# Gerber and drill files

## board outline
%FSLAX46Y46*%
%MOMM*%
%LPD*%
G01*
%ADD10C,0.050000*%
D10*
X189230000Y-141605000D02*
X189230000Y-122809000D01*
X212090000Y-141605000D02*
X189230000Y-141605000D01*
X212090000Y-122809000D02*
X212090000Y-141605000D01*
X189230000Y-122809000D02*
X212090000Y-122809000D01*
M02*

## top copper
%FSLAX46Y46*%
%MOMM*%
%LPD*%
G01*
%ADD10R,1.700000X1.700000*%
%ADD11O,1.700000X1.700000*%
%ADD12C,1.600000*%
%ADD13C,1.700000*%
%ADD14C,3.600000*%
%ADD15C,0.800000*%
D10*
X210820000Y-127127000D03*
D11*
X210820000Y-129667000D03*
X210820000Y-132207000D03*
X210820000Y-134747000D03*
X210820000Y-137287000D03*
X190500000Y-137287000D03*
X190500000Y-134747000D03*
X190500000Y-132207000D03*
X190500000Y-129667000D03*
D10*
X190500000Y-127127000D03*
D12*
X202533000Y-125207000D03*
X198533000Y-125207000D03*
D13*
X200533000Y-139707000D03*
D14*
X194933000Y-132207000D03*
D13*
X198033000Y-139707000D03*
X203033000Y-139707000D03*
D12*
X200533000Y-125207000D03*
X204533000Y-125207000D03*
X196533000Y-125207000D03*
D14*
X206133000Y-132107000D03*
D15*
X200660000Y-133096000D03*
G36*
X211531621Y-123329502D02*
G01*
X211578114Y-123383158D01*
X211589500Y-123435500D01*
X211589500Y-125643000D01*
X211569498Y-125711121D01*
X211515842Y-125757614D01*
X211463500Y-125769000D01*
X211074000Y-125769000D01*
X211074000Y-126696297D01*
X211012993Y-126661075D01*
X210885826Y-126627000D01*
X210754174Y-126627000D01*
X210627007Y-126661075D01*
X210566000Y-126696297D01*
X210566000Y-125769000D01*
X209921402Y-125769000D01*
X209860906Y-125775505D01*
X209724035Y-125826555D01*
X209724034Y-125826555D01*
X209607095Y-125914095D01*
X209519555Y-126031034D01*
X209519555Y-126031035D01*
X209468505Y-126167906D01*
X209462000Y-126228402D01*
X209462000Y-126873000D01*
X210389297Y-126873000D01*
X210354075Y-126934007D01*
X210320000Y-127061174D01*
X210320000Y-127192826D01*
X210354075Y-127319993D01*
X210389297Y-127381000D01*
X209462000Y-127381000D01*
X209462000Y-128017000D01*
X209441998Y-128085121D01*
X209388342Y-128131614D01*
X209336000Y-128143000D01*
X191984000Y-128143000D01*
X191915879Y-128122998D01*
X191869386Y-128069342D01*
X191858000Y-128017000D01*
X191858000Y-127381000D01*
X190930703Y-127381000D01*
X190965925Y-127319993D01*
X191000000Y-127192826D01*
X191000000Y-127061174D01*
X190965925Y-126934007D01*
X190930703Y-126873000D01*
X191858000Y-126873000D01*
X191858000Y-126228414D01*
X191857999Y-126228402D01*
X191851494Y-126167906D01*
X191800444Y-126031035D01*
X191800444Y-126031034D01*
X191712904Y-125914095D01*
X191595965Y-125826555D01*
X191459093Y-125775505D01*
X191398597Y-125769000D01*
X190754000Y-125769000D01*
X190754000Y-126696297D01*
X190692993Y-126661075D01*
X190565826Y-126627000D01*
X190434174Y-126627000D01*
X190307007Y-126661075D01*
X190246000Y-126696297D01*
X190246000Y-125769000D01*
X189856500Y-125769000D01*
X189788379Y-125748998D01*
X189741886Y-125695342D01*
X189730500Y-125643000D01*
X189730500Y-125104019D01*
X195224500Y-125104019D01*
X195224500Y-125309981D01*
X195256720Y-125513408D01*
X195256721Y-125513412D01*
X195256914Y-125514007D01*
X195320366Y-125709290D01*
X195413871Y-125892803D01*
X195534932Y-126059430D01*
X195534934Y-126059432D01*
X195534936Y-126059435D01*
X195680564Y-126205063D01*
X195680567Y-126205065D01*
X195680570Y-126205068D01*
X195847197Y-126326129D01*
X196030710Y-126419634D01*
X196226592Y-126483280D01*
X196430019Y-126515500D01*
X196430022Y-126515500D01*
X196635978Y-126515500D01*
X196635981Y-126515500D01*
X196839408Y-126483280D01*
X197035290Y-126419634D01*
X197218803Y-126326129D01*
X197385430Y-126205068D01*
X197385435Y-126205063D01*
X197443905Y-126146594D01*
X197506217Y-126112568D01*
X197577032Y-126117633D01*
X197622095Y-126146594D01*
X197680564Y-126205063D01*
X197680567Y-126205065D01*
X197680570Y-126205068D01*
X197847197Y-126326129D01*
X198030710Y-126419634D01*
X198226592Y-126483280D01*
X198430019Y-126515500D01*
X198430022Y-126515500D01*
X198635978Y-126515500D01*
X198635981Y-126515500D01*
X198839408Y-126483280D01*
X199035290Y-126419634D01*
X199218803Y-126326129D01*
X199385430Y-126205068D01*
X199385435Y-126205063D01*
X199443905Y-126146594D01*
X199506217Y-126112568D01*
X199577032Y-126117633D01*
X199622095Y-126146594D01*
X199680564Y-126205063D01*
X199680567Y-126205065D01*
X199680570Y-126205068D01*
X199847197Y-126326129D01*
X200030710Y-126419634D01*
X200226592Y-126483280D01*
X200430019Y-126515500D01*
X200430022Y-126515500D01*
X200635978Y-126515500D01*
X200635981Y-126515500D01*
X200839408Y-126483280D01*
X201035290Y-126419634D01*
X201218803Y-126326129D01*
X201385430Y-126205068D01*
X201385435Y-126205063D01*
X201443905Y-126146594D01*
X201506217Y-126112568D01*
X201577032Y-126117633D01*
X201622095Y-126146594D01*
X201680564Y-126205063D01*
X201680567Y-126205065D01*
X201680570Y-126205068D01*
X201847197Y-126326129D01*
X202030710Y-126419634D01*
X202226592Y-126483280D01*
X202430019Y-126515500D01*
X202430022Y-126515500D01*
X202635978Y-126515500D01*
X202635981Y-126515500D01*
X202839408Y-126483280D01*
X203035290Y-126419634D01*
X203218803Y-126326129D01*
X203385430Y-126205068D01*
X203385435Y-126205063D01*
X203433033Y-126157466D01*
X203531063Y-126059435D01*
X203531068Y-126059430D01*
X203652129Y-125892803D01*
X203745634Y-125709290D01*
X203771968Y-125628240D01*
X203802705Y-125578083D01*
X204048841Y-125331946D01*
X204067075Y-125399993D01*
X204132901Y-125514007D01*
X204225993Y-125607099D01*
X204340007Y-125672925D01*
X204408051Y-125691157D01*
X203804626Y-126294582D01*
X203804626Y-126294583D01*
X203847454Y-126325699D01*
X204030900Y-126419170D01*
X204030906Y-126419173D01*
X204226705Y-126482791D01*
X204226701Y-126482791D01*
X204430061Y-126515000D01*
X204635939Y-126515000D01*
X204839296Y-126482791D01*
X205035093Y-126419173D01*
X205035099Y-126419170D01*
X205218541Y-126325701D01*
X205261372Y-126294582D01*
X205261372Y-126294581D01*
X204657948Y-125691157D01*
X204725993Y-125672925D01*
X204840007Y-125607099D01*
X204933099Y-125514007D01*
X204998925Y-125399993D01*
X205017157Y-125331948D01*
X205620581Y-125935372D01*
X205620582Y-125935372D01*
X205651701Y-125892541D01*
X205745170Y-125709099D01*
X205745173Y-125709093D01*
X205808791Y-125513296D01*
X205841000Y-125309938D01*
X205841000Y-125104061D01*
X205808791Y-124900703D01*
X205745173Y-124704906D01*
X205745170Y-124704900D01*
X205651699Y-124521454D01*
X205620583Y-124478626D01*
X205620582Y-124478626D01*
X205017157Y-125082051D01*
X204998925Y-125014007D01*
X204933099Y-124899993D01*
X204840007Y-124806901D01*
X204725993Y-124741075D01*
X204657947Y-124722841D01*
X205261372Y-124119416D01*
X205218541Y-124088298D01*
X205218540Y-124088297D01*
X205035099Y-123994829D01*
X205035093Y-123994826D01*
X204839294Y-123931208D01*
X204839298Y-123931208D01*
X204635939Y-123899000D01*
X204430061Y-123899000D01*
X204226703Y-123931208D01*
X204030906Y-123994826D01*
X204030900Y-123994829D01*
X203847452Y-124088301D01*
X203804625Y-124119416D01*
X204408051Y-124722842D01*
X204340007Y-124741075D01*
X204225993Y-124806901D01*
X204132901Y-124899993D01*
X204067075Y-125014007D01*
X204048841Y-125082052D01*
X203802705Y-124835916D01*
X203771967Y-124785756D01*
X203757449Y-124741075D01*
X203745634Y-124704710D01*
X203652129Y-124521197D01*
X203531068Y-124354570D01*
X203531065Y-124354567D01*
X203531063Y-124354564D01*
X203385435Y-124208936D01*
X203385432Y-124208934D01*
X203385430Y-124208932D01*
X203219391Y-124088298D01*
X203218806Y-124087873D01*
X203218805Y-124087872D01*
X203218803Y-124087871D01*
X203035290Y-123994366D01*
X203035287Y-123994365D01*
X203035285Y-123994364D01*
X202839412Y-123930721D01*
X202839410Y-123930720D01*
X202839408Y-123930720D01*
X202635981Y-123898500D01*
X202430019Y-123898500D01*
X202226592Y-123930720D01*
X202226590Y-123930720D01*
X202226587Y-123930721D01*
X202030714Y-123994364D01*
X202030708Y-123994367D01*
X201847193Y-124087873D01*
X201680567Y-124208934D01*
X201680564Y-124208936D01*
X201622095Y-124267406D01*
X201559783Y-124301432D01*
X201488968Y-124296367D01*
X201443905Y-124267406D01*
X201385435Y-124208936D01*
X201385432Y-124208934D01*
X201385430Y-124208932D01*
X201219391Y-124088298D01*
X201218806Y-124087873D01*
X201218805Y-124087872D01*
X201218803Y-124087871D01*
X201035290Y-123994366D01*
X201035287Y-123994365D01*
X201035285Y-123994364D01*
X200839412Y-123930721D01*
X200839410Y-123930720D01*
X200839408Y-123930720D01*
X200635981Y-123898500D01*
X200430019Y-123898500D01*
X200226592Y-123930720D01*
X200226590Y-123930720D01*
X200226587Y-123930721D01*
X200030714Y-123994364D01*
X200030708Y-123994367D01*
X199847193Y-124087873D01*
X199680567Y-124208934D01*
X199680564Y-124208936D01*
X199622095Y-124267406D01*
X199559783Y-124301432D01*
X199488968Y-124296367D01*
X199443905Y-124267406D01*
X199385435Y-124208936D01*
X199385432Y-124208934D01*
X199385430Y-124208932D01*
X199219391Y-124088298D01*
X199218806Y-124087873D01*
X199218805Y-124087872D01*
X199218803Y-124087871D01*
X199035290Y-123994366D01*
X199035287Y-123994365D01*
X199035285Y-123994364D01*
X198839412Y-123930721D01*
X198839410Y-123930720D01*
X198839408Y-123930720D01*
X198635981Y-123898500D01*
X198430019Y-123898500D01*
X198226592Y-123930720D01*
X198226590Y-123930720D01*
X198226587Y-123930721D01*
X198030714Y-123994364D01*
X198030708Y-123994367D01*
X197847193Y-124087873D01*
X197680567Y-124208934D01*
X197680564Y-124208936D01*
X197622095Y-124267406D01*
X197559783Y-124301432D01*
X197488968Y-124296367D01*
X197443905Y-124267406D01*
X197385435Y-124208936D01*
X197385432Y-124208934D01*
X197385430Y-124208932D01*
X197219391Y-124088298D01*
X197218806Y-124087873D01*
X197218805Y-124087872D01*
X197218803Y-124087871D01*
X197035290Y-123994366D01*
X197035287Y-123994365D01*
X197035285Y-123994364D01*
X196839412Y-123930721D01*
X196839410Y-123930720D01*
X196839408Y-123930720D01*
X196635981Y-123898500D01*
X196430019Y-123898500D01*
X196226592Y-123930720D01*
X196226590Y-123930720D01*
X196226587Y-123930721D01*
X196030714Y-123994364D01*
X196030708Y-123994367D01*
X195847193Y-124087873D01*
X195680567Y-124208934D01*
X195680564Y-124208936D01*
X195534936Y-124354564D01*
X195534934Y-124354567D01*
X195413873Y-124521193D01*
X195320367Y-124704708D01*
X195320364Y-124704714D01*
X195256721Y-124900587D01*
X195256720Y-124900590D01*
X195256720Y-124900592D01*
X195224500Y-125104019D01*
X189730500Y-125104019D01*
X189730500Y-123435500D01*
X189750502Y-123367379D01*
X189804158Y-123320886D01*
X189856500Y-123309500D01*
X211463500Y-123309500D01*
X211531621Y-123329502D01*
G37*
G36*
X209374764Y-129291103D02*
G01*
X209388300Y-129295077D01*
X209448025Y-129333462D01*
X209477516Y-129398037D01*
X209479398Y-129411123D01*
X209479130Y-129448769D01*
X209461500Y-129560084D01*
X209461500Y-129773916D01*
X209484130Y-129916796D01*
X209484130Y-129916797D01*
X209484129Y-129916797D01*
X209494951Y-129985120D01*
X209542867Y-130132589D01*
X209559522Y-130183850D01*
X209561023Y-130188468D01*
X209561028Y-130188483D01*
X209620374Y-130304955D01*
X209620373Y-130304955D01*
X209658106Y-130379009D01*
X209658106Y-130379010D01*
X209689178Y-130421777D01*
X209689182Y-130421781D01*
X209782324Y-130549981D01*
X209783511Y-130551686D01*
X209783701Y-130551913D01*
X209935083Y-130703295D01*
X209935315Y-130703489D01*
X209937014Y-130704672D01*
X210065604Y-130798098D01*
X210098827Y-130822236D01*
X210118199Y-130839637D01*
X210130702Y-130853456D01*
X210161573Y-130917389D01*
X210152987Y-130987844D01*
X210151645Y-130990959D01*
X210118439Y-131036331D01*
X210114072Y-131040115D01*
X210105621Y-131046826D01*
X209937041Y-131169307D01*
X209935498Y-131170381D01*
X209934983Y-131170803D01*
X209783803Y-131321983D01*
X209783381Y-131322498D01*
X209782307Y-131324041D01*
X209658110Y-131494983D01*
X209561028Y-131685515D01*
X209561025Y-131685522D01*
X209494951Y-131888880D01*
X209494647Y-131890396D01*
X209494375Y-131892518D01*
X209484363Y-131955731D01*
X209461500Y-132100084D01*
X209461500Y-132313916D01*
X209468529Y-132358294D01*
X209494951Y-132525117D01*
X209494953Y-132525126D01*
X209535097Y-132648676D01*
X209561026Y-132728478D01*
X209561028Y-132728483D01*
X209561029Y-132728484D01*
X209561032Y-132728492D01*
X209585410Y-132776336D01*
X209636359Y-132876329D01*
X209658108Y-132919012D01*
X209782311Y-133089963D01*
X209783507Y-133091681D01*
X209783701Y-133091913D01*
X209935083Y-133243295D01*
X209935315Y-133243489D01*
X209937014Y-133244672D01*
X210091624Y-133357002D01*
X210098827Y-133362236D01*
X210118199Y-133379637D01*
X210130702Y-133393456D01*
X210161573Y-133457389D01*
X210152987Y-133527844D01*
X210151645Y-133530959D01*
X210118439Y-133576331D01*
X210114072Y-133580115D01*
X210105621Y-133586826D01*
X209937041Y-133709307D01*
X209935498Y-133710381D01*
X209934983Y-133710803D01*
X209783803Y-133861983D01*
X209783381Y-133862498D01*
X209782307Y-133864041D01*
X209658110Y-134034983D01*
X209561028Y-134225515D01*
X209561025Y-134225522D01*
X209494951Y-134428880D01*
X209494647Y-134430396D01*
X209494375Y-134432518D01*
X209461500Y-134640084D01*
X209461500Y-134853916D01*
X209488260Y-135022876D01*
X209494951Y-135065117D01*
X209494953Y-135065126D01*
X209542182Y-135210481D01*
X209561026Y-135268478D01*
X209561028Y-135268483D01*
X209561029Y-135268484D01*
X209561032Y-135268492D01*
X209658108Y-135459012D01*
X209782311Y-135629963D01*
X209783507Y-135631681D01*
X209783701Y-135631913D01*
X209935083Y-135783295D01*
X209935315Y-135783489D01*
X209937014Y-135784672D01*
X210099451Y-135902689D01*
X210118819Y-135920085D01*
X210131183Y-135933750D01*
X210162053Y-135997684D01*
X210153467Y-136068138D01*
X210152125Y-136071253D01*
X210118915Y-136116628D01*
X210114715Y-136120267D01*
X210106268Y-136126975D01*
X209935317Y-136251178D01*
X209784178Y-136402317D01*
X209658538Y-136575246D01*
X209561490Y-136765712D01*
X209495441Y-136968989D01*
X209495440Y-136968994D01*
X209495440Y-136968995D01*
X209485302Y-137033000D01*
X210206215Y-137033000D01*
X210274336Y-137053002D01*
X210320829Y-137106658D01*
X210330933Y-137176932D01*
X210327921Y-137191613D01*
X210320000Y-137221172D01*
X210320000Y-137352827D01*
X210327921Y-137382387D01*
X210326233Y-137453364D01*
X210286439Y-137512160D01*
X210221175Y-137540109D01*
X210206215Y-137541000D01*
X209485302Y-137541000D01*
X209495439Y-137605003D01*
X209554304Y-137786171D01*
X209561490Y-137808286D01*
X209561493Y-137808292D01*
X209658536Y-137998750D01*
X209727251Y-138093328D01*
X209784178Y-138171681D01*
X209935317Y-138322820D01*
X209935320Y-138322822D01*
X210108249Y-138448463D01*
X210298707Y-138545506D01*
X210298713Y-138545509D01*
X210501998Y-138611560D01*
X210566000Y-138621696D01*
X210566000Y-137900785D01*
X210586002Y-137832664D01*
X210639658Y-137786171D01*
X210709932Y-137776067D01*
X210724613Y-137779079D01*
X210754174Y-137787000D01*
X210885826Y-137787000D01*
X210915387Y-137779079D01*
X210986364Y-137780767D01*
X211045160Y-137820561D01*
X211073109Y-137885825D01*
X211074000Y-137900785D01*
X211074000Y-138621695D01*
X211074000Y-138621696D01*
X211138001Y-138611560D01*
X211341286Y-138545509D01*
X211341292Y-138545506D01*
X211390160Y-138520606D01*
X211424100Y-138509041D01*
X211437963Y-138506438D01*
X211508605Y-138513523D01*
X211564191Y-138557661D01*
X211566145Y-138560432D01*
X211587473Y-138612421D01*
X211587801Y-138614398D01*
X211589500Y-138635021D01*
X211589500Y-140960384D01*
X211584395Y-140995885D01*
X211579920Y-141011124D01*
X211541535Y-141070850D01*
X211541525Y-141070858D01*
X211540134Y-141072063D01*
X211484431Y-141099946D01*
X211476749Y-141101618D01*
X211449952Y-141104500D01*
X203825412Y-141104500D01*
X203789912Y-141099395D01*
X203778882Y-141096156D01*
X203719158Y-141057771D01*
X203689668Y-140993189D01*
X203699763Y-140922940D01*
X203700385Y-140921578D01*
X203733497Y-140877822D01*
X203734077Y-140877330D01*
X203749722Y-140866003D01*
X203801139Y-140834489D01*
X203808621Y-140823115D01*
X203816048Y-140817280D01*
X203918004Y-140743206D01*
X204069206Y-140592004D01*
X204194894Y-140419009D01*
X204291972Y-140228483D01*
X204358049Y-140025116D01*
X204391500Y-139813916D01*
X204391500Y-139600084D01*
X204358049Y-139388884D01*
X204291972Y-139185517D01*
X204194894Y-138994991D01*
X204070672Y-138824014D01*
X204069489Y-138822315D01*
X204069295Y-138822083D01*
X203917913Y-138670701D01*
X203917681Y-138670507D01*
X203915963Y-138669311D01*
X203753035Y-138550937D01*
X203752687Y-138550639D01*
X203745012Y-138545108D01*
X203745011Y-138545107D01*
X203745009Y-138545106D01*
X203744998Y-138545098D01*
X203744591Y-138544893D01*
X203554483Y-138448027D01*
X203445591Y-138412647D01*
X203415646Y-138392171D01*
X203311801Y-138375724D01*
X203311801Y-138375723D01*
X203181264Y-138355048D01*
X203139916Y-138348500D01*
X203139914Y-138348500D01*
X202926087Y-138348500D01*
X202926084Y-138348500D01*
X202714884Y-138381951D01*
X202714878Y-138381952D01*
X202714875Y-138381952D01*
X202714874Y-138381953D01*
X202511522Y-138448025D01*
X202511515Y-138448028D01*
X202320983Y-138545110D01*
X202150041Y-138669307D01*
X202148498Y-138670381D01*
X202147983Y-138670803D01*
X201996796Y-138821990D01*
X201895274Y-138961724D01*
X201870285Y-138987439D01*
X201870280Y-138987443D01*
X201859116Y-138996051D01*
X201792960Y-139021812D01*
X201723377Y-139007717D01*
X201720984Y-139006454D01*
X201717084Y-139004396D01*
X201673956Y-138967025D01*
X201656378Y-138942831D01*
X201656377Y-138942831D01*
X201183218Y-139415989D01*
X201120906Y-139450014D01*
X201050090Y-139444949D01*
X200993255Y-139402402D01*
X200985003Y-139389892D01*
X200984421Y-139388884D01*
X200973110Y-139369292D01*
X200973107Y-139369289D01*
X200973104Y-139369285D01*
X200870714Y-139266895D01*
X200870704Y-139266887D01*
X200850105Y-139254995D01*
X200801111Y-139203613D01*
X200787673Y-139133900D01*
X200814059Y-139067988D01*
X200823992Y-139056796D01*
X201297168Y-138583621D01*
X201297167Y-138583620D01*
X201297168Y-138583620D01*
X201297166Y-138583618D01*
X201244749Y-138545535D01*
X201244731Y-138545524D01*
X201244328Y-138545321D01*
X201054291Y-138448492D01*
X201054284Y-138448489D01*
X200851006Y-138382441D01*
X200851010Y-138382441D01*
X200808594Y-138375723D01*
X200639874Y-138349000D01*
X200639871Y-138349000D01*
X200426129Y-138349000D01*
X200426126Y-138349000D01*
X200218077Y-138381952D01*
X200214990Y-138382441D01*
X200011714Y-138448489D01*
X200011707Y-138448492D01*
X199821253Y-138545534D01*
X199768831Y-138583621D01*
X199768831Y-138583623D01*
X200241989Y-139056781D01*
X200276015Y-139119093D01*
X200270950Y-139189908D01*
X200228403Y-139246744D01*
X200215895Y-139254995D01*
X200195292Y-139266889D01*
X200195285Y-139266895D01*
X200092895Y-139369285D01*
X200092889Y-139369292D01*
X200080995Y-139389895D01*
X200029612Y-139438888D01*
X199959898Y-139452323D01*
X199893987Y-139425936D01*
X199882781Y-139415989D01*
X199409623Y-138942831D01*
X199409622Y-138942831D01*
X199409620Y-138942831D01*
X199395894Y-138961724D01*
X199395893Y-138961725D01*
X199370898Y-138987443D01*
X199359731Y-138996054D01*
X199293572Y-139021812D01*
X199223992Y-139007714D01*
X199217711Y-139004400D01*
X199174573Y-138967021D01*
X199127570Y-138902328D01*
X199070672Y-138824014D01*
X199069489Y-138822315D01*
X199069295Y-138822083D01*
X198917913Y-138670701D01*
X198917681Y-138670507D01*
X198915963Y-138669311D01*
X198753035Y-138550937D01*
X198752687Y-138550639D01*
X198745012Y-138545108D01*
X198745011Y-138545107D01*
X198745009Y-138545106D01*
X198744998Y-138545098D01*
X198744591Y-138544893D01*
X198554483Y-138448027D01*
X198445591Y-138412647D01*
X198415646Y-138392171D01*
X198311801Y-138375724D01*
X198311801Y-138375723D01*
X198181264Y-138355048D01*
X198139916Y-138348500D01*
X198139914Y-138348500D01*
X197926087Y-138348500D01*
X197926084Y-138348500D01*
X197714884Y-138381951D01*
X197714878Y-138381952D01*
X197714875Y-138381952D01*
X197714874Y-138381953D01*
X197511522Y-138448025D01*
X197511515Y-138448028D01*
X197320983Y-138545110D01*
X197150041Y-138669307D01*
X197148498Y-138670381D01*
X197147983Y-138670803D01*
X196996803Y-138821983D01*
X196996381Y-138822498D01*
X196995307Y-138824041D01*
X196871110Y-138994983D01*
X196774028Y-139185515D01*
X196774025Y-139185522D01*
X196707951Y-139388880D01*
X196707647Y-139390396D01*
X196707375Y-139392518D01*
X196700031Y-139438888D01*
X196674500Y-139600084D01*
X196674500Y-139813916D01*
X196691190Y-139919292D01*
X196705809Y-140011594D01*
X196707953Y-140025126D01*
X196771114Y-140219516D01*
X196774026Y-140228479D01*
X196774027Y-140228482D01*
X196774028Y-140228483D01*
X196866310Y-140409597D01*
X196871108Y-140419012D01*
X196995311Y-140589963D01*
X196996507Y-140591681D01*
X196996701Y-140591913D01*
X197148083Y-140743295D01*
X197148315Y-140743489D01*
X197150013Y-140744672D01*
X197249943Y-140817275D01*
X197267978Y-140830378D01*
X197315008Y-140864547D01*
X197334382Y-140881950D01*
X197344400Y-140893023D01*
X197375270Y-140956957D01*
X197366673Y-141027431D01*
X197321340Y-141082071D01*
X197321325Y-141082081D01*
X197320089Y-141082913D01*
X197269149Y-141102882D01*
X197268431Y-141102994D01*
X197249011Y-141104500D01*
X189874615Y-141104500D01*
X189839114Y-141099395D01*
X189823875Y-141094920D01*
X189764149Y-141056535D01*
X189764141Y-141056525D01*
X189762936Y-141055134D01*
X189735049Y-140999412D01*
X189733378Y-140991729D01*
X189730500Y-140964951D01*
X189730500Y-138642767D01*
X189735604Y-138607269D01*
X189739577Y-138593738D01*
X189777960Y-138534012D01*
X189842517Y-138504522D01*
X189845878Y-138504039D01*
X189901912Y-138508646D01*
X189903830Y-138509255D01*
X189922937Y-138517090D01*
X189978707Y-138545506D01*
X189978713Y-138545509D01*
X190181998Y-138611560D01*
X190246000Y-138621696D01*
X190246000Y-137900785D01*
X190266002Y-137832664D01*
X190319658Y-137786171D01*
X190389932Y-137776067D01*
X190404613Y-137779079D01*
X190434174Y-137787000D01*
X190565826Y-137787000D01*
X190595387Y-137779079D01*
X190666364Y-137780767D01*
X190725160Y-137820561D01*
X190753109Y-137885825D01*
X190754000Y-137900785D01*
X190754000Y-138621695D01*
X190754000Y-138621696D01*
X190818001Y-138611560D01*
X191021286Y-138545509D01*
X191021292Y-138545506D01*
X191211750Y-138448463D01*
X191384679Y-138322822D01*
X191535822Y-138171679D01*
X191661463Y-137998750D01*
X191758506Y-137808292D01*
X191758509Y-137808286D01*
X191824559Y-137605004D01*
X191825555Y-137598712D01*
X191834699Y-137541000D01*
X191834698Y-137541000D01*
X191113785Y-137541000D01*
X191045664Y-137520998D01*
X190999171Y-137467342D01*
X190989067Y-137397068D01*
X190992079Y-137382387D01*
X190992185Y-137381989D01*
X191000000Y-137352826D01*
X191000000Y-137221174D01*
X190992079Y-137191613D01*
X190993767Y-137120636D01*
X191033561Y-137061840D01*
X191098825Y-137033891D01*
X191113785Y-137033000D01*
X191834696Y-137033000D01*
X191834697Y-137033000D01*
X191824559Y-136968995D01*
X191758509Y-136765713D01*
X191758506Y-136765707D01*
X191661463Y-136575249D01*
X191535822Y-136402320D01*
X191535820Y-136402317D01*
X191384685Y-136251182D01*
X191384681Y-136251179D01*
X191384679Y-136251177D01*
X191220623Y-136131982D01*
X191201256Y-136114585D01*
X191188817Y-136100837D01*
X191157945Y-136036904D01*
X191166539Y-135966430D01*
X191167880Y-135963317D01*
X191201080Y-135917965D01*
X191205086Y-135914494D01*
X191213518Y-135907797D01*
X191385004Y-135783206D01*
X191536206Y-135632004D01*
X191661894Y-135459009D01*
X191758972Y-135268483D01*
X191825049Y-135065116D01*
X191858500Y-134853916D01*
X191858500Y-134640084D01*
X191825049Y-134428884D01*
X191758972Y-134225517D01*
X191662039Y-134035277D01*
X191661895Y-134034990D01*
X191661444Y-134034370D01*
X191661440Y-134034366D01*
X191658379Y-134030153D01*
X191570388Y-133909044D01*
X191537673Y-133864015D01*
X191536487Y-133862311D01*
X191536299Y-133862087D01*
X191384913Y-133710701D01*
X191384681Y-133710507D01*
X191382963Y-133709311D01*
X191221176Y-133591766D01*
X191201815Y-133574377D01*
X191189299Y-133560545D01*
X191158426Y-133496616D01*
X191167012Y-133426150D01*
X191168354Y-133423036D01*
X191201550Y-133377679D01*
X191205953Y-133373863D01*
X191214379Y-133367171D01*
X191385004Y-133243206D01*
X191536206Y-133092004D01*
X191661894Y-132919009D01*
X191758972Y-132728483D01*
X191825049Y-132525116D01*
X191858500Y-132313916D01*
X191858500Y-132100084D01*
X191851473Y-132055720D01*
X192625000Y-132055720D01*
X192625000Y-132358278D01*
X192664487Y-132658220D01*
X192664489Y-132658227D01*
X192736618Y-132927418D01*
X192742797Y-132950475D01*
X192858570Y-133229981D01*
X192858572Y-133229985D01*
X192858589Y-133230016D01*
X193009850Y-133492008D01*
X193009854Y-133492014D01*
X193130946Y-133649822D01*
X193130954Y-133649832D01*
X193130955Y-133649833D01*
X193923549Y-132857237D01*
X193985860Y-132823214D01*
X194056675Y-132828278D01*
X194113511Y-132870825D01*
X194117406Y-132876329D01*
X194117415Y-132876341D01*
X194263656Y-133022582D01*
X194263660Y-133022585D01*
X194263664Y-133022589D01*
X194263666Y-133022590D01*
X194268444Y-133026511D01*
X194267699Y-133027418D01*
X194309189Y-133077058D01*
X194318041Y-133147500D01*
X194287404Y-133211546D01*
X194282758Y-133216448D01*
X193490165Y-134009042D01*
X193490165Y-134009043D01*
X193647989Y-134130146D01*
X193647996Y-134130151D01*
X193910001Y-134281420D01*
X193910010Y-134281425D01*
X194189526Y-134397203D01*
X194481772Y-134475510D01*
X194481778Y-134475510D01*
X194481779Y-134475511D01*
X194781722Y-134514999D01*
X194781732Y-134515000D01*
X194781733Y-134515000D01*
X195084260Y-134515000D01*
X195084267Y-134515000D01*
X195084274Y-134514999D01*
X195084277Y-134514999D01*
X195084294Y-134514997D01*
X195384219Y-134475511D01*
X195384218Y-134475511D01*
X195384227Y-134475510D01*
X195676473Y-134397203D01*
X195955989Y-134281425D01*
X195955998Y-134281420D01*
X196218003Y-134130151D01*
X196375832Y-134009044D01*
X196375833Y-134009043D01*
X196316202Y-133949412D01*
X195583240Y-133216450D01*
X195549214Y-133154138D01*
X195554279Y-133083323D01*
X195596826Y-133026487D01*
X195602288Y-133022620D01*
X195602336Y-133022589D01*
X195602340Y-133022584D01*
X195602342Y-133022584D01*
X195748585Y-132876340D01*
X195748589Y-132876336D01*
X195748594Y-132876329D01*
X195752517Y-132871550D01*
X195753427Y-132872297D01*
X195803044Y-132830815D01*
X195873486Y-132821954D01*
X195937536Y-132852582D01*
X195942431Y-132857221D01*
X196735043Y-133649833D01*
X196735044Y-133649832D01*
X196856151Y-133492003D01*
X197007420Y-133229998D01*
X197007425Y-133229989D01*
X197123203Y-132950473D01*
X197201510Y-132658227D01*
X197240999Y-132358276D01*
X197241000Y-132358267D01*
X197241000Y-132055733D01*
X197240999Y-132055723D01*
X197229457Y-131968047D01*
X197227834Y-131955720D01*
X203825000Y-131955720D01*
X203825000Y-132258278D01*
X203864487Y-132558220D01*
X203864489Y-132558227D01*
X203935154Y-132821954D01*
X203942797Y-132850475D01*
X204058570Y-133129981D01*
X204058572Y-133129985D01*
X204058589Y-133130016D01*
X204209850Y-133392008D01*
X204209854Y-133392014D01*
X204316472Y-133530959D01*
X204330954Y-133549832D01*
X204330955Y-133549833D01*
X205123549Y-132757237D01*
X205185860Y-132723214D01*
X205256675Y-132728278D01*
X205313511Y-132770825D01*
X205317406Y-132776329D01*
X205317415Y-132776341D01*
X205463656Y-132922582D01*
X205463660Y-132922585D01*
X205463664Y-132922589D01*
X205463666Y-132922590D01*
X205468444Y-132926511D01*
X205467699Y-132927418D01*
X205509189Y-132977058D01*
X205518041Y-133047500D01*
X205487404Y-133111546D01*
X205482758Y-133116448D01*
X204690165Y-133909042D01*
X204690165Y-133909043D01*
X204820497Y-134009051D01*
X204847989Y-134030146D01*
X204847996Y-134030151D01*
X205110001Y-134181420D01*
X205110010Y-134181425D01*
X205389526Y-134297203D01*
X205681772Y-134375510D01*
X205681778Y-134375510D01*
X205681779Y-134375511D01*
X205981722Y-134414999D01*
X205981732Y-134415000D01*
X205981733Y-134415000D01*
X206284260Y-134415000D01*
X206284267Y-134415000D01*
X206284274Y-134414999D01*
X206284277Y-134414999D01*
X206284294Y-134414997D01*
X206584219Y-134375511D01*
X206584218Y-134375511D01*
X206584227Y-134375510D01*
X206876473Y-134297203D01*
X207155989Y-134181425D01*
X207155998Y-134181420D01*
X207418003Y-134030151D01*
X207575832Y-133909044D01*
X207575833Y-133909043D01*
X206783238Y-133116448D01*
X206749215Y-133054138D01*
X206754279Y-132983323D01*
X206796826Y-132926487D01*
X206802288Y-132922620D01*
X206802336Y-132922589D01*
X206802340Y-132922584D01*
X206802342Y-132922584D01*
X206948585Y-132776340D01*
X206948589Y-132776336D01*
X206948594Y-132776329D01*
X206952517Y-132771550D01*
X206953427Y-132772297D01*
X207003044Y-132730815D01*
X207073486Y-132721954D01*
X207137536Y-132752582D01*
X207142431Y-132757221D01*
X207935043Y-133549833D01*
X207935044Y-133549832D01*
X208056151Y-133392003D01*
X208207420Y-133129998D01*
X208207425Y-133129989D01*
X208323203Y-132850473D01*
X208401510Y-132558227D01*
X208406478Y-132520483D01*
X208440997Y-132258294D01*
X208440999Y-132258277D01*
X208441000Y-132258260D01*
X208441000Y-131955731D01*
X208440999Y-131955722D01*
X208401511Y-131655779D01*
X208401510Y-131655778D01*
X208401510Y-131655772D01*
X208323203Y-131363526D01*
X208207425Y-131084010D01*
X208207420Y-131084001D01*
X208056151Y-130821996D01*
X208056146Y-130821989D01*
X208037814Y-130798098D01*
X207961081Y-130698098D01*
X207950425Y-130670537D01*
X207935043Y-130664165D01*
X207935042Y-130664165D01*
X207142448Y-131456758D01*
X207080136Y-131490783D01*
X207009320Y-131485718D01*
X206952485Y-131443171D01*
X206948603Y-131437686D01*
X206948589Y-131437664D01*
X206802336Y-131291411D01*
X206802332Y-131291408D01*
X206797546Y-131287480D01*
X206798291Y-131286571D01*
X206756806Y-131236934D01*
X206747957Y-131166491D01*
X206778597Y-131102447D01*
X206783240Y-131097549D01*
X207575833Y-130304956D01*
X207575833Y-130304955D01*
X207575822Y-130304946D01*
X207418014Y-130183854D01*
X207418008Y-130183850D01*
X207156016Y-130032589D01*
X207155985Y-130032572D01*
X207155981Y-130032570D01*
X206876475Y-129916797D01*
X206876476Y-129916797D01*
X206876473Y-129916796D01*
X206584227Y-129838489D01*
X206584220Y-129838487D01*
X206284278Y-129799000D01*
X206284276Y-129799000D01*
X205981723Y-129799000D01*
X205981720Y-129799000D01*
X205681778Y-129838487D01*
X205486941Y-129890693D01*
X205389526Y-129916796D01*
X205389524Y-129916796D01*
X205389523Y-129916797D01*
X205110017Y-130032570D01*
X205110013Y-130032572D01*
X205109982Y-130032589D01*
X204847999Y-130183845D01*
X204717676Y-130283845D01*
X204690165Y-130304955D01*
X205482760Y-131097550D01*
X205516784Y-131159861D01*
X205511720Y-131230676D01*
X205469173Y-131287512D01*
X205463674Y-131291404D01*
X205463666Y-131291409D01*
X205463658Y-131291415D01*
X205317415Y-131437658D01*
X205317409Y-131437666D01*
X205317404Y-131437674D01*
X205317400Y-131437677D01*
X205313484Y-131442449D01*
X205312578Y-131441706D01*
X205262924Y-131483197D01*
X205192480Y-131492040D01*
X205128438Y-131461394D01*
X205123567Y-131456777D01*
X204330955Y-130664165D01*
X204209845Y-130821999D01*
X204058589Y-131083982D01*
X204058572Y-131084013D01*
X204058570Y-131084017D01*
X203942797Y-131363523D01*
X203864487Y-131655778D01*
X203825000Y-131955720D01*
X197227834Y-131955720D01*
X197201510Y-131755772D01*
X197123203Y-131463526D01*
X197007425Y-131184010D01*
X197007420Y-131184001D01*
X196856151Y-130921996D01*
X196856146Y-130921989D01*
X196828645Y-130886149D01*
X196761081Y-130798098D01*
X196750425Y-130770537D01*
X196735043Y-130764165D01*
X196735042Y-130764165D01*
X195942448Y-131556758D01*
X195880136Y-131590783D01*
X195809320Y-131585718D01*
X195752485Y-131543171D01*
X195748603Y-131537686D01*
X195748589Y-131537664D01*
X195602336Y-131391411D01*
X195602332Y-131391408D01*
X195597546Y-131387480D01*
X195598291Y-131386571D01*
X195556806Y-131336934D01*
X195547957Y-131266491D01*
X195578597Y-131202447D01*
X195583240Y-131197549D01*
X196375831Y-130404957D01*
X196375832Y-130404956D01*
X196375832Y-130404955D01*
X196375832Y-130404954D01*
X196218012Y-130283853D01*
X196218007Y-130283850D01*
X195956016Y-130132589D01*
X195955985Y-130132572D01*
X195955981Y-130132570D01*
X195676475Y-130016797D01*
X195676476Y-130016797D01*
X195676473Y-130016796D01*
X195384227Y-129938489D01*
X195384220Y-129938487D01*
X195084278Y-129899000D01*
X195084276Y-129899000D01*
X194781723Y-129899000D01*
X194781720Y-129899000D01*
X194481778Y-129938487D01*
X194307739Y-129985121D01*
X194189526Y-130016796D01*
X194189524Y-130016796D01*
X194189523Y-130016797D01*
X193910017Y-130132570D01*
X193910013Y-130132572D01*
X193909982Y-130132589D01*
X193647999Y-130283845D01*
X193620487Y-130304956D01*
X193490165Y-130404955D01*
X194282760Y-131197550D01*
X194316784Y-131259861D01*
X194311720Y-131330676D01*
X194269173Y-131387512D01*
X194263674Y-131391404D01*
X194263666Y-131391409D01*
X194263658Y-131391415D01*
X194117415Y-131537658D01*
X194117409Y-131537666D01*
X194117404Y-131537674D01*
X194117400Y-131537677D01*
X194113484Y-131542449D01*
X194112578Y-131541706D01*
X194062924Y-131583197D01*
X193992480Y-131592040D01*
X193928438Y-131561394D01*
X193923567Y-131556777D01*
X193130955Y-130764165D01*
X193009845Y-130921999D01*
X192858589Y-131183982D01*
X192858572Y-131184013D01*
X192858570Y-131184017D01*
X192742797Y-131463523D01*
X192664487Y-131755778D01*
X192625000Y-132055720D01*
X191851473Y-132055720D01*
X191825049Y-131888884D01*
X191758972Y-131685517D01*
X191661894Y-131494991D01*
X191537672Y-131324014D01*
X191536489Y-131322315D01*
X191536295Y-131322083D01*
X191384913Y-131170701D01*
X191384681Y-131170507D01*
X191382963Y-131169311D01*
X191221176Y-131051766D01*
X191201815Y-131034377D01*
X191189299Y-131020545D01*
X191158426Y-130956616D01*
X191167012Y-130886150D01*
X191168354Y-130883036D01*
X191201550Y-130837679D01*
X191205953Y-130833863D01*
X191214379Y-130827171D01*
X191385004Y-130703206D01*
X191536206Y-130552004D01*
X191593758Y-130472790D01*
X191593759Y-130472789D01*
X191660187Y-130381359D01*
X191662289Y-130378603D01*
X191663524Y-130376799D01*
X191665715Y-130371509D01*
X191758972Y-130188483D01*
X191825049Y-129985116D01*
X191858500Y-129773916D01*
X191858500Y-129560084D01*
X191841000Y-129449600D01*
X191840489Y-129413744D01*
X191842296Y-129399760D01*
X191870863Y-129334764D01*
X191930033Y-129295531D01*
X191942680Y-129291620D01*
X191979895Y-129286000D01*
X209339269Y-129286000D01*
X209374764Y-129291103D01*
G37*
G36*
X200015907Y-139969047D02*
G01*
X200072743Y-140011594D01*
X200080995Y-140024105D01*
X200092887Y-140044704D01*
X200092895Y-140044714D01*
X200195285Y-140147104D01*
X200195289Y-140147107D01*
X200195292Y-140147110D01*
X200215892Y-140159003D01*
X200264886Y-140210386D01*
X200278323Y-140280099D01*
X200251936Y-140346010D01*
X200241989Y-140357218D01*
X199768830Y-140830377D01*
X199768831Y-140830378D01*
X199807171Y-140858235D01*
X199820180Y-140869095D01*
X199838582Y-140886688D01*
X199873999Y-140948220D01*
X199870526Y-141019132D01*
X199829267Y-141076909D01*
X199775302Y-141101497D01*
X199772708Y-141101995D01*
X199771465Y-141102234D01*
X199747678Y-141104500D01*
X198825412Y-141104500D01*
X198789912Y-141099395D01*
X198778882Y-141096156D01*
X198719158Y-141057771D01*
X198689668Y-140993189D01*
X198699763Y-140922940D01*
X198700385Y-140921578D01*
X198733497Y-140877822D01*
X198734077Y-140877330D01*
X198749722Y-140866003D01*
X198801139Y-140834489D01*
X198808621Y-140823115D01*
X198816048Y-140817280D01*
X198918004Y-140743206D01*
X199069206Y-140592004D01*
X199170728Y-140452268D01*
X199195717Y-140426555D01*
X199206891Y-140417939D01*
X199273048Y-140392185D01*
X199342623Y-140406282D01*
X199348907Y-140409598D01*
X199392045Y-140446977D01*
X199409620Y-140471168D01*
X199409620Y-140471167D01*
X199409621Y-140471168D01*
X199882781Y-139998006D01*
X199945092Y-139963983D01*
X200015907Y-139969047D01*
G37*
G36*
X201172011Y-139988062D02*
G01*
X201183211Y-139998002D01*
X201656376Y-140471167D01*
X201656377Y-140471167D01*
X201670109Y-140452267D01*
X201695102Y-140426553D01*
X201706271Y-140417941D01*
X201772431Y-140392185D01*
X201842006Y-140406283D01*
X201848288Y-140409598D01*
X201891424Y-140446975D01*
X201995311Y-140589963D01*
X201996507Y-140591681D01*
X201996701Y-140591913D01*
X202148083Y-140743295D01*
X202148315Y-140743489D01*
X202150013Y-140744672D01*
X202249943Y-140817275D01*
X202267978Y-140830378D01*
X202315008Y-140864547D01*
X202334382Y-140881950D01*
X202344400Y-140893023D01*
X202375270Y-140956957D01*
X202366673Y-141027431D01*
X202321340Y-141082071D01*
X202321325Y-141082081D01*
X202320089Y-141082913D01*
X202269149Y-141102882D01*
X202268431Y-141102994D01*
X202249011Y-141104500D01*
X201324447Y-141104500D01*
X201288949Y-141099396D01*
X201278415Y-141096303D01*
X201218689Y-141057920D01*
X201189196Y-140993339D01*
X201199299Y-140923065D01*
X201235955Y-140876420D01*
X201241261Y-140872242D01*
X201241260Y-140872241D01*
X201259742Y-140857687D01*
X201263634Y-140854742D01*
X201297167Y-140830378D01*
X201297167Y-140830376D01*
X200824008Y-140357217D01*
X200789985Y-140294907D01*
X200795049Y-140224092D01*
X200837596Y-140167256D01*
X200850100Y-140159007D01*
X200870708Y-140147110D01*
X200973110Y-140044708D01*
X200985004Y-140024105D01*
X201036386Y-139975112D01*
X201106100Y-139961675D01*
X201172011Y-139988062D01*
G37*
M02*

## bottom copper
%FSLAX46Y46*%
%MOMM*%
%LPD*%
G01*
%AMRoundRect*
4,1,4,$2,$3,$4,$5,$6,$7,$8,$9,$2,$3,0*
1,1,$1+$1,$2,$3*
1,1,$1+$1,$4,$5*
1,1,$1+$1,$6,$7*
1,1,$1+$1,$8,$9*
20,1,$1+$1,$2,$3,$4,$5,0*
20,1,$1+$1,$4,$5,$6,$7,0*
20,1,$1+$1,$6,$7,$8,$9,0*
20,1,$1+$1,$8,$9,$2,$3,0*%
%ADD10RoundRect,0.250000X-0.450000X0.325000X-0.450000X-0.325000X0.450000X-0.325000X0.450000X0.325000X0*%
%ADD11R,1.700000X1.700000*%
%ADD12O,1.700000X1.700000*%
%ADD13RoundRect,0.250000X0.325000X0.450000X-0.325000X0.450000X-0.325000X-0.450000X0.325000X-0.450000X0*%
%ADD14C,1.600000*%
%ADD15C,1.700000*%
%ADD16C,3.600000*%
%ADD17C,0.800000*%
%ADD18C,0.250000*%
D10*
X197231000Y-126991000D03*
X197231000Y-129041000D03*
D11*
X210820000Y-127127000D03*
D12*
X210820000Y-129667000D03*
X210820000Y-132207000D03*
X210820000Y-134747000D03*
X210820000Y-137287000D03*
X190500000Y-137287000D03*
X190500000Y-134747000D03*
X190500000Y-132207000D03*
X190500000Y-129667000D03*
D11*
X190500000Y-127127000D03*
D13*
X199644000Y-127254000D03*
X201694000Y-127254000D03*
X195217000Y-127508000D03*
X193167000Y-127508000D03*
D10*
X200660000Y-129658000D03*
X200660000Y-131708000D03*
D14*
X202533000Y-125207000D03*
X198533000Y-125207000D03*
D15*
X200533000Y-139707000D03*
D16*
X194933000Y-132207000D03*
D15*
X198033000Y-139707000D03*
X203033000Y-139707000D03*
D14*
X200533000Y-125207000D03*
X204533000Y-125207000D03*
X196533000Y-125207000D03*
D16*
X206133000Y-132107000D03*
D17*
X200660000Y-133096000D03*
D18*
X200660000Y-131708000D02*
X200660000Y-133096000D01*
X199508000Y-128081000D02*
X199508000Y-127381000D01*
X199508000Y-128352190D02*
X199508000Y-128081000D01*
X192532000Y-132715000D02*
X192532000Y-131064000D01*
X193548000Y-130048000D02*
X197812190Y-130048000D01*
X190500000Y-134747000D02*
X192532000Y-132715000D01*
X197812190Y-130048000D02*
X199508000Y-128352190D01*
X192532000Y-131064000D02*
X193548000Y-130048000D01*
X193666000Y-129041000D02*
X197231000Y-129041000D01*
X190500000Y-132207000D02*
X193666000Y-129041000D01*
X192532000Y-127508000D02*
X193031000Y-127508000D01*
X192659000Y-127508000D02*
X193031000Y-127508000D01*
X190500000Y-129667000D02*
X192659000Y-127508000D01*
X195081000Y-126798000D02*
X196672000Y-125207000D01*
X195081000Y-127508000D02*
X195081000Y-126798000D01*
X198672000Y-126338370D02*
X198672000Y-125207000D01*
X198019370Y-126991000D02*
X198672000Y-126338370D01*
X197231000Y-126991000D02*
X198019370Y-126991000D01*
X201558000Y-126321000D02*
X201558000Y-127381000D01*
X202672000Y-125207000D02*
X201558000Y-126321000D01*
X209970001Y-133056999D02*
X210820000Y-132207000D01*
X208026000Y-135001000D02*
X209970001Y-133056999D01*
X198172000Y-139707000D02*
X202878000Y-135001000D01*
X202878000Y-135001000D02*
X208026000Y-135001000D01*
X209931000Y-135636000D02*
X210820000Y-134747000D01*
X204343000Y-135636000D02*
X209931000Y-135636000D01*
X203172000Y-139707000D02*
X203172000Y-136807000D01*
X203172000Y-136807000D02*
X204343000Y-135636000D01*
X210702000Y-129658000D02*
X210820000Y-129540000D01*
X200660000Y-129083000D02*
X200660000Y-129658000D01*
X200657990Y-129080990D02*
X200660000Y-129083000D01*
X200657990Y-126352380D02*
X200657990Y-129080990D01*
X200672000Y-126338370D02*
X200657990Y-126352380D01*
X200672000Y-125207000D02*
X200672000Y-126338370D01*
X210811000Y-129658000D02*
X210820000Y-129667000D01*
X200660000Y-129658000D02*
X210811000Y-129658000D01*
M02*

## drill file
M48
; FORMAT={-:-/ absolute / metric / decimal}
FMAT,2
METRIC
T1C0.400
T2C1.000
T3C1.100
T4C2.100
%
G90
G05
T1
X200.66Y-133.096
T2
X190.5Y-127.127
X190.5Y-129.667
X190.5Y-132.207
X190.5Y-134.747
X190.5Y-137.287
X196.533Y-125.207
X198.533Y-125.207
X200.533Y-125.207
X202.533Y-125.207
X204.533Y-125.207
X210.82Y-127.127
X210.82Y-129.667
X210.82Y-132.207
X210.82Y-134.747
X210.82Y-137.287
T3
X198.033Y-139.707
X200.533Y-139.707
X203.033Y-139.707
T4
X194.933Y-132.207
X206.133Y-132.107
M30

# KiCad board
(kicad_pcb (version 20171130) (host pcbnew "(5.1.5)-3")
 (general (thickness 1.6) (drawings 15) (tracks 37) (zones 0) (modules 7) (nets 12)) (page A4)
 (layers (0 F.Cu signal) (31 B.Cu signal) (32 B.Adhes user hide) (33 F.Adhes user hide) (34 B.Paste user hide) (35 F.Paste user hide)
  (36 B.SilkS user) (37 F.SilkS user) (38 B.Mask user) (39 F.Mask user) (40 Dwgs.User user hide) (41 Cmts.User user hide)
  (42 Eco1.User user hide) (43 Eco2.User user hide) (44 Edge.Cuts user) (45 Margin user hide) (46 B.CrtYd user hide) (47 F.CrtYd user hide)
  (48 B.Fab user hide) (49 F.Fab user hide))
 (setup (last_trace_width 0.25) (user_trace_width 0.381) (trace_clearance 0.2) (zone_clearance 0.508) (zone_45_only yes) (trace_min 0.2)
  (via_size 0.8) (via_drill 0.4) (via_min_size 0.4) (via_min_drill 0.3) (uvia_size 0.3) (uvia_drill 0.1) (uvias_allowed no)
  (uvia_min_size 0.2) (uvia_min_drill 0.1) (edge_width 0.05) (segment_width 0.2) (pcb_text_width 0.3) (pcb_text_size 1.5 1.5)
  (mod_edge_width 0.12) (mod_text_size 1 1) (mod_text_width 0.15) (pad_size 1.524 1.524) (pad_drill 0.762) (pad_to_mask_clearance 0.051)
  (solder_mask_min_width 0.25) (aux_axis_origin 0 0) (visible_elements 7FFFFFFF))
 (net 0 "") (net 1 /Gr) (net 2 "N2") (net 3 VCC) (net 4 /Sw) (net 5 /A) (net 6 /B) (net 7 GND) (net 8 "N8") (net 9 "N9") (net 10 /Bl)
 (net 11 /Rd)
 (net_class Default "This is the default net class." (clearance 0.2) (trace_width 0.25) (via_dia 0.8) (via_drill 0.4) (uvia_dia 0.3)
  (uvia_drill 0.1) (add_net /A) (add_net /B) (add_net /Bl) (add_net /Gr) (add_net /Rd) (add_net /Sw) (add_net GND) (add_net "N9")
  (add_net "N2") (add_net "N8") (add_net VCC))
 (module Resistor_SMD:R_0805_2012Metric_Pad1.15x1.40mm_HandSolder (layer B.Cu) (at 197.231 128.016 270)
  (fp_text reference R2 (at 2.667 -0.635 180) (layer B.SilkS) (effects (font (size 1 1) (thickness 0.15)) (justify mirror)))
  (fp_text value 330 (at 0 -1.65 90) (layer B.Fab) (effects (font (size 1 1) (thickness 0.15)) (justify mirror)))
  (pad 1 smd roundrect (at -1.025 0 270) (size 1.15 1.4) (layers B.Cu B.Paste B.Mask) (roundrect_rratio 0.217391) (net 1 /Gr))
  (pad 2 smd roundrect (at 1.025 0 270) (size 1.15 1.4) (layers B.Cu B.Paste B.Mask) (roundrect_rratio 0.217391) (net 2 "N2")))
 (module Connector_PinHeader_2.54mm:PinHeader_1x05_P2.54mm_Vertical (layer F.Cu) (at 210.82 127.127)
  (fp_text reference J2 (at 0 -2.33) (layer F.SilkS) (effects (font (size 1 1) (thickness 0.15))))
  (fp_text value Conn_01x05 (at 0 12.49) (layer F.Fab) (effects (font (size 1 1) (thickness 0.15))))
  (pad 1 thru_hole rect (at 0 0) (size 1.7 1.7) (drill 1) (layers *.Cu *.Mask) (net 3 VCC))
  (pad 2 thru_hole oval (at 0 2.54) (size 1.7 1.7) (drill 1) (layers *.Cu *.Mask) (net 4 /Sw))
  (pad 3 thru_hole oval (at 0 5.08) (size 1.7 1.7) (drill 1) (layers *.Cu *.Mask) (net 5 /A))
  (pad 4 thru_hole oval (at 0 7.62) (size 1.7 1.7) (drill 1) (layers *.Cu *.Mask) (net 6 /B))
  (pad 5 thru_hole oval (at 0 10.16) (size 1.7 1.7) (drill 1) (layers *.Cu *.Mask) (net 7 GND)))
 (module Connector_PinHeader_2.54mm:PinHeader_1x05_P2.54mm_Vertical (layer F.Cu) (at 190.5 127.127)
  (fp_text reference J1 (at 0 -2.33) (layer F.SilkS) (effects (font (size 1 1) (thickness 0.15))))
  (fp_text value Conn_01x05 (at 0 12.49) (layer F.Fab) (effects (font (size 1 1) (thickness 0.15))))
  (pad 5 thru_hole oval (at 0 10.16) (size 1.7 1.7) (drill 1) (layers *.Cu *.Mask) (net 7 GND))
  (pad 4 thru_hole oval (at 0 7.62) (size 1.7 1.7) (drill 1) (layers *.Cu *.Mask) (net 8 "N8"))
  (pad 3 thru_hole oval (at 0 5.08) (size 1.7 1.7) (drill 1) (layers *.Cu *.Mask) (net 2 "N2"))
  (pad 2 thru_hole oval (at 0 2.54) (size 1.7 1.7) (drill 1) (layers *.Cu *.Mask) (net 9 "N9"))
  (pad 1 thru_hole rect (at 0 0) (size 1.7 1.7) (drill 1) (layers *.Cu *.Mask) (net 3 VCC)))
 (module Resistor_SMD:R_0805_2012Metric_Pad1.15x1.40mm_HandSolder (layer B.Cu) (at 200.669 127.254 180)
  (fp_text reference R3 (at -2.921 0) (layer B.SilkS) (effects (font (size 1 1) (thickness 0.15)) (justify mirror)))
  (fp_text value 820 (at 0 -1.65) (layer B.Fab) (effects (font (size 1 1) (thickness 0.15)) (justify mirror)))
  (pad 2 smd roundrect (at 1.025 0 180) (size 1.15 1.4) (layers B.Cu B.Paste B.Mask) (roundrect_rratio 0.217391) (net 8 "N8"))
  (pad 1 smd roundrect (at -1.025 0 180) (size 1.15 1.4) (layers B.Cu B.Paste B.Mask) (roundrect_rratio 0.217391) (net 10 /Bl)))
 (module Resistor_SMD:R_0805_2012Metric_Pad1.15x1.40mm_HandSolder (layer B.Cu) (at 194.192 127.508 180)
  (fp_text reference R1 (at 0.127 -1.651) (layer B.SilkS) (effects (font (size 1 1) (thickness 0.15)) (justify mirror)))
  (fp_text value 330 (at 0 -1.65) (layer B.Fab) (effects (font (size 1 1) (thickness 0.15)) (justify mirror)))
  (pad 1 smd roundrect (at -1.025 0 180) (size 1.15 1.4) (layers B.Cu B.Paste B.Mask) (roundrect_rratio 0.217391) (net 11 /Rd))
  (pad 2 smd roundrect (at 1.025 0 180) (size 1.15 1.4) (layers B.Cu B.Paste B.Mask) (roundrect_rratio 0.217391) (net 9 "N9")))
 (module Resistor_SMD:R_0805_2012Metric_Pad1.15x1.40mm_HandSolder (layer B.Cu) (at 200.66 130.683 270)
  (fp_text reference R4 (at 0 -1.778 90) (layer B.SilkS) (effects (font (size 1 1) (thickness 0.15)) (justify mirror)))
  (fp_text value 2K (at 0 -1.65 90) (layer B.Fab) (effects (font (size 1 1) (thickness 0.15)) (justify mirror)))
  (pad 1 smd roundrect (at -1.025 0 270) (size 1.15 1.4) (layers B.Cu B.Paste B.Mask) (roundrect_rratio 0.217391) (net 4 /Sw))
  (pad 2 smd roundrect (at 1.025 0 270) (size 1.15 1.4) (layers B.Cu B.Paste B.Mask) (roundrect_rratio 0.217391) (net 7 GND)))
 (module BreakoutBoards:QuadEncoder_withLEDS (layer F.Cu) (at 200.533 132.207)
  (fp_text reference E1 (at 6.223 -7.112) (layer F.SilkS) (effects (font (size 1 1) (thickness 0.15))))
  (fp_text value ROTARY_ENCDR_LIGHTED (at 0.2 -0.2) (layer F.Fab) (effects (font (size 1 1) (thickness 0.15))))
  (pad 4 thru_hole circle (at 2 -7) (size 1.6 1.6) (drill 1) (layers *.Cu *.Mask F.SilkS) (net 10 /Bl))
  (pad 2 thru_hole circle (at -2 -7) (size 1.6 1.6) (drill 1) (layers *.Cu *.Mask F.SilkS) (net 1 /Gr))
  (pad 7 thru_hole circle (at 0 7.5) (size 1.7 1.7) (drill 1.1) (layers *.Cu *.Mask F.SilkS) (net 7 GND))
  (pad 9 thru_hole circle (at -5.6 0) (size 3.6 3.6) (drill 2.1) (layers *.Cu *.Mask F.SilkS) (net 7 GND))
  (pad 8 thru_hole circle (at -2.5 7.5) (size 1.7 1.7) (drill 1.1) (layers *.Cu *.Mask F.SilkS) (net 5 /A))
  (pad 6 thru_hole circle (at 2.5 7.5) (size 1.7 1.7) (drill 1.1) (layers *.Cu *.Mask F.SilkS) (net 6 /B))
  (pad 3 thru_hole circle (at 0 -7) (size 1.6 1.6) (drill 1) (layers *.Cu *.Mask F.SilkS) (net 4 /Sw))
  (pad 5 thru_hole circle (at 4 -7) (size 1.6 1.6) (drill 1) (layers *.Cu *.Mask F.SilkS) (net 3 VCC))
  (pad 1 thru_hole circle (at -4 -7) (size 1.6 1.6) (drill 1) (layers *.Cu *.Mask F.SilkS) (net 11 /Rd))
  (pad 10 thru_hole circle (at 5.6 -0.1) (size 3.6 3.6) (drill 2.1) (layers *.Cu *.Mask F.SilkS) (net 7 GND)))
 (gr_line (start 189.23 141.605) (end 189.23 122.809) (layer Edge.Cuts) (width 0.05))
 (gr_line (start 212.09 141.605) (end 189.23 141.605) (layer Edge.Cuts) (width 0.05))
 (gr_line (start 212.09 122.809) (end 212.09 141.605) (layer Edge.Cuts) (width 0.05))
 (gr_line (start 189.23 122.809) (end 212.09 122.809) (layer Edge.Cuts) (width 0.05))
 (via (at 200.66 133.096) (size 0.8) (drill 0.4) (layers F.Cu B.Cu) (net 7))
 (segment (start 200.66 131.708) (end 200.66 133.096) (width 0.25) (layer B.Cu) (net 7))
 (segment (start 199.508 128.081) (end 199.508 127.381) (width 0.25) (layer B.Cu) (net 8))
 (segment (start 199.508 128.35219) (end 199.508 128.081) (width 0.25) (layer B.Cu) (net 8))
 (segment (start 192.532 132.715) (end 192.532 131.064) (width 0.25) (layer B.Cu) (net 8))
 (segment (start 193.548 130.048) (end 197.81219 130.048) (width 0.25) (layer B.Cu) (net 8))
 (segment (start 190.5 134.747) (end 192.532 132.715) (width 0.25) (layer B.Cu) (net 8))
 (segment (start 197.81219 130.048) (end 199.508 128.35219) (width 0.25) (layer B.Cu) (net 8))
 (segment (start 192.532 131.064) (end 193.548 130.048) (width 0.25) (layer B.Cu) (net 8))
 (segment (start 193.666 129.041) (end 197.231 129.041) (width 0.25) (layer B.Cu) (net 2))
 (segment (start 190.5 132.207) (end 193.666 129.041) (width 0.25) (layer B.Cu) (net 2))
 (segment (start 192.532 127.508) (end 193.031 127.508) (width 0.25) (layer B.Cu) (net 9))
 (segment (start 192.659 127.508) (end 193.031 127.508) (width 0.25) (layer B.Cu) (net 9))
 (segment (start 190.5 129.667) (end 192.659 127.508) (width 0.25) (layer B.Cu) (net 9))
 (segment (start 195.081 126.798) (end 196.672 125.207) (width 0.25) (layer B.Cu) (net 11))
 (segment (start 195.081 127.508) (end 195.081 126.798) (width 0.25) (layer B.Cu) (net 11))
 (segment (start 198.672 126.33837) (end 198.672 125.207) (width 0.25) (layer B.Cu) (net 1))
 (segment (start 198.01937 126.991) (end 198.672 126.33837) (width 0.25) (layer B.Cu) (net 1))
 (segment (start 197.231 126.991) (end 198.01937 126.991) (width 0.25) (layer B.Cu) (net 1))
 (segment (start 201.558 126.321) (end 201.558 127.381) (width 0.25) (layer B.Cu) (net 10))
 (segment (start 202.672 125.207) (end 201.558 126.321) (width 0.25) (layer B.Cu) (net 10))
 (segment (start 209.970001 133.056999) (end 210.82 132.207) (width 0.25) (layer B.Cu) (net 5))
 (segment (start 208.026 135.001) (end 209.970001 133.056999) (width 0.25) (layer B.Cu) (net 5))
 (segment (start 198.172 139.707) (end 202.878 135.001) (width 0.25) (layer B.Cu) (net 5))
 (segment (start 202.878 135.001) (end 208.026 135.001) (width 0.25) (layer B.Cu) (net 5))
 (segment (start 209.931 135.636) (end 210.82 134.747) (width 0.25) (layer B.Cu) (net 6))
 (segment (start 204.343 135.636) (end 209.931 135.636) (width 0.25) (layer B.Cu) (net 6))
 (segment (start 203.172 139.707) (end 203.172 136.807) (width 0.25) (layer B.Cu) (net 6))
 (segment (start 203.172 136.807) (end 204.343 135.636) (width 0.25) (layer B.Cu) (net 6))
 (segment (start 210.702 129.658) (end 210.82 129.54) (width 0.25) (layer B.Cu) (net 4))
 (segment (start 200.66 129.083) (end 200.66 129.658) (width 0.25) (layer B.Cu) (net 4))
 (segment (start 200.65799 129.08099) (end 200.66 129.083) (width 0.25) (layer B.Cu) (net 4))
 (segment (start 200.65799 126.35238) (end 200.65799 129.08099) (width 0.25) (layer B.Cu) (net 4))
 (segment (start 200.672 126.33837) (end 200.65799 126.35238) (width 0.25) (layer B.Cu) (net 4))
 (segment (start 200.672 125.207) (end 200.672 126.33837) (width 0.25) (layer B.Cu) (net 4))
 (segment (start 210.811 129.658) (end 210.82 129.667) (width 0.25) (layer B.Cu) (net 4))
 (segment (start 200.66 129.658) (end 210.811 129.658) (width 0.25) (layer B.Cu) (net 4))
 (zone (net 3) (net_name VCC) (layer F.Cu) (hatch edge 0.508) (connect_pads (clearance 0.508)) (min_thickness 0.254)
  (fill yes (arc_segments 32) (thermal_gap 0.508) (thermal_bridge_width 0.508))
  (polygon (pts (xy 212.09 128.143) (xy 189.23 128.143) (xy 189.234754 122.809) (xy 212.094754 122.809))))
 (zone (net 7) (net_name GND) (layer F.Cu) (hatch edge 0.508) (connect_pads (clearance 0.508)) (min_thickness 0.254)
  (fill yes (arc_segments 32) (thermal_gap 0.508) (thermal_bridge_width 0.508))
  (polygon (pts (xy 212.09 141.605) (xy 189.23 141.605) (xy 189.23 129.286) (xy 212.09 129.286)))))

